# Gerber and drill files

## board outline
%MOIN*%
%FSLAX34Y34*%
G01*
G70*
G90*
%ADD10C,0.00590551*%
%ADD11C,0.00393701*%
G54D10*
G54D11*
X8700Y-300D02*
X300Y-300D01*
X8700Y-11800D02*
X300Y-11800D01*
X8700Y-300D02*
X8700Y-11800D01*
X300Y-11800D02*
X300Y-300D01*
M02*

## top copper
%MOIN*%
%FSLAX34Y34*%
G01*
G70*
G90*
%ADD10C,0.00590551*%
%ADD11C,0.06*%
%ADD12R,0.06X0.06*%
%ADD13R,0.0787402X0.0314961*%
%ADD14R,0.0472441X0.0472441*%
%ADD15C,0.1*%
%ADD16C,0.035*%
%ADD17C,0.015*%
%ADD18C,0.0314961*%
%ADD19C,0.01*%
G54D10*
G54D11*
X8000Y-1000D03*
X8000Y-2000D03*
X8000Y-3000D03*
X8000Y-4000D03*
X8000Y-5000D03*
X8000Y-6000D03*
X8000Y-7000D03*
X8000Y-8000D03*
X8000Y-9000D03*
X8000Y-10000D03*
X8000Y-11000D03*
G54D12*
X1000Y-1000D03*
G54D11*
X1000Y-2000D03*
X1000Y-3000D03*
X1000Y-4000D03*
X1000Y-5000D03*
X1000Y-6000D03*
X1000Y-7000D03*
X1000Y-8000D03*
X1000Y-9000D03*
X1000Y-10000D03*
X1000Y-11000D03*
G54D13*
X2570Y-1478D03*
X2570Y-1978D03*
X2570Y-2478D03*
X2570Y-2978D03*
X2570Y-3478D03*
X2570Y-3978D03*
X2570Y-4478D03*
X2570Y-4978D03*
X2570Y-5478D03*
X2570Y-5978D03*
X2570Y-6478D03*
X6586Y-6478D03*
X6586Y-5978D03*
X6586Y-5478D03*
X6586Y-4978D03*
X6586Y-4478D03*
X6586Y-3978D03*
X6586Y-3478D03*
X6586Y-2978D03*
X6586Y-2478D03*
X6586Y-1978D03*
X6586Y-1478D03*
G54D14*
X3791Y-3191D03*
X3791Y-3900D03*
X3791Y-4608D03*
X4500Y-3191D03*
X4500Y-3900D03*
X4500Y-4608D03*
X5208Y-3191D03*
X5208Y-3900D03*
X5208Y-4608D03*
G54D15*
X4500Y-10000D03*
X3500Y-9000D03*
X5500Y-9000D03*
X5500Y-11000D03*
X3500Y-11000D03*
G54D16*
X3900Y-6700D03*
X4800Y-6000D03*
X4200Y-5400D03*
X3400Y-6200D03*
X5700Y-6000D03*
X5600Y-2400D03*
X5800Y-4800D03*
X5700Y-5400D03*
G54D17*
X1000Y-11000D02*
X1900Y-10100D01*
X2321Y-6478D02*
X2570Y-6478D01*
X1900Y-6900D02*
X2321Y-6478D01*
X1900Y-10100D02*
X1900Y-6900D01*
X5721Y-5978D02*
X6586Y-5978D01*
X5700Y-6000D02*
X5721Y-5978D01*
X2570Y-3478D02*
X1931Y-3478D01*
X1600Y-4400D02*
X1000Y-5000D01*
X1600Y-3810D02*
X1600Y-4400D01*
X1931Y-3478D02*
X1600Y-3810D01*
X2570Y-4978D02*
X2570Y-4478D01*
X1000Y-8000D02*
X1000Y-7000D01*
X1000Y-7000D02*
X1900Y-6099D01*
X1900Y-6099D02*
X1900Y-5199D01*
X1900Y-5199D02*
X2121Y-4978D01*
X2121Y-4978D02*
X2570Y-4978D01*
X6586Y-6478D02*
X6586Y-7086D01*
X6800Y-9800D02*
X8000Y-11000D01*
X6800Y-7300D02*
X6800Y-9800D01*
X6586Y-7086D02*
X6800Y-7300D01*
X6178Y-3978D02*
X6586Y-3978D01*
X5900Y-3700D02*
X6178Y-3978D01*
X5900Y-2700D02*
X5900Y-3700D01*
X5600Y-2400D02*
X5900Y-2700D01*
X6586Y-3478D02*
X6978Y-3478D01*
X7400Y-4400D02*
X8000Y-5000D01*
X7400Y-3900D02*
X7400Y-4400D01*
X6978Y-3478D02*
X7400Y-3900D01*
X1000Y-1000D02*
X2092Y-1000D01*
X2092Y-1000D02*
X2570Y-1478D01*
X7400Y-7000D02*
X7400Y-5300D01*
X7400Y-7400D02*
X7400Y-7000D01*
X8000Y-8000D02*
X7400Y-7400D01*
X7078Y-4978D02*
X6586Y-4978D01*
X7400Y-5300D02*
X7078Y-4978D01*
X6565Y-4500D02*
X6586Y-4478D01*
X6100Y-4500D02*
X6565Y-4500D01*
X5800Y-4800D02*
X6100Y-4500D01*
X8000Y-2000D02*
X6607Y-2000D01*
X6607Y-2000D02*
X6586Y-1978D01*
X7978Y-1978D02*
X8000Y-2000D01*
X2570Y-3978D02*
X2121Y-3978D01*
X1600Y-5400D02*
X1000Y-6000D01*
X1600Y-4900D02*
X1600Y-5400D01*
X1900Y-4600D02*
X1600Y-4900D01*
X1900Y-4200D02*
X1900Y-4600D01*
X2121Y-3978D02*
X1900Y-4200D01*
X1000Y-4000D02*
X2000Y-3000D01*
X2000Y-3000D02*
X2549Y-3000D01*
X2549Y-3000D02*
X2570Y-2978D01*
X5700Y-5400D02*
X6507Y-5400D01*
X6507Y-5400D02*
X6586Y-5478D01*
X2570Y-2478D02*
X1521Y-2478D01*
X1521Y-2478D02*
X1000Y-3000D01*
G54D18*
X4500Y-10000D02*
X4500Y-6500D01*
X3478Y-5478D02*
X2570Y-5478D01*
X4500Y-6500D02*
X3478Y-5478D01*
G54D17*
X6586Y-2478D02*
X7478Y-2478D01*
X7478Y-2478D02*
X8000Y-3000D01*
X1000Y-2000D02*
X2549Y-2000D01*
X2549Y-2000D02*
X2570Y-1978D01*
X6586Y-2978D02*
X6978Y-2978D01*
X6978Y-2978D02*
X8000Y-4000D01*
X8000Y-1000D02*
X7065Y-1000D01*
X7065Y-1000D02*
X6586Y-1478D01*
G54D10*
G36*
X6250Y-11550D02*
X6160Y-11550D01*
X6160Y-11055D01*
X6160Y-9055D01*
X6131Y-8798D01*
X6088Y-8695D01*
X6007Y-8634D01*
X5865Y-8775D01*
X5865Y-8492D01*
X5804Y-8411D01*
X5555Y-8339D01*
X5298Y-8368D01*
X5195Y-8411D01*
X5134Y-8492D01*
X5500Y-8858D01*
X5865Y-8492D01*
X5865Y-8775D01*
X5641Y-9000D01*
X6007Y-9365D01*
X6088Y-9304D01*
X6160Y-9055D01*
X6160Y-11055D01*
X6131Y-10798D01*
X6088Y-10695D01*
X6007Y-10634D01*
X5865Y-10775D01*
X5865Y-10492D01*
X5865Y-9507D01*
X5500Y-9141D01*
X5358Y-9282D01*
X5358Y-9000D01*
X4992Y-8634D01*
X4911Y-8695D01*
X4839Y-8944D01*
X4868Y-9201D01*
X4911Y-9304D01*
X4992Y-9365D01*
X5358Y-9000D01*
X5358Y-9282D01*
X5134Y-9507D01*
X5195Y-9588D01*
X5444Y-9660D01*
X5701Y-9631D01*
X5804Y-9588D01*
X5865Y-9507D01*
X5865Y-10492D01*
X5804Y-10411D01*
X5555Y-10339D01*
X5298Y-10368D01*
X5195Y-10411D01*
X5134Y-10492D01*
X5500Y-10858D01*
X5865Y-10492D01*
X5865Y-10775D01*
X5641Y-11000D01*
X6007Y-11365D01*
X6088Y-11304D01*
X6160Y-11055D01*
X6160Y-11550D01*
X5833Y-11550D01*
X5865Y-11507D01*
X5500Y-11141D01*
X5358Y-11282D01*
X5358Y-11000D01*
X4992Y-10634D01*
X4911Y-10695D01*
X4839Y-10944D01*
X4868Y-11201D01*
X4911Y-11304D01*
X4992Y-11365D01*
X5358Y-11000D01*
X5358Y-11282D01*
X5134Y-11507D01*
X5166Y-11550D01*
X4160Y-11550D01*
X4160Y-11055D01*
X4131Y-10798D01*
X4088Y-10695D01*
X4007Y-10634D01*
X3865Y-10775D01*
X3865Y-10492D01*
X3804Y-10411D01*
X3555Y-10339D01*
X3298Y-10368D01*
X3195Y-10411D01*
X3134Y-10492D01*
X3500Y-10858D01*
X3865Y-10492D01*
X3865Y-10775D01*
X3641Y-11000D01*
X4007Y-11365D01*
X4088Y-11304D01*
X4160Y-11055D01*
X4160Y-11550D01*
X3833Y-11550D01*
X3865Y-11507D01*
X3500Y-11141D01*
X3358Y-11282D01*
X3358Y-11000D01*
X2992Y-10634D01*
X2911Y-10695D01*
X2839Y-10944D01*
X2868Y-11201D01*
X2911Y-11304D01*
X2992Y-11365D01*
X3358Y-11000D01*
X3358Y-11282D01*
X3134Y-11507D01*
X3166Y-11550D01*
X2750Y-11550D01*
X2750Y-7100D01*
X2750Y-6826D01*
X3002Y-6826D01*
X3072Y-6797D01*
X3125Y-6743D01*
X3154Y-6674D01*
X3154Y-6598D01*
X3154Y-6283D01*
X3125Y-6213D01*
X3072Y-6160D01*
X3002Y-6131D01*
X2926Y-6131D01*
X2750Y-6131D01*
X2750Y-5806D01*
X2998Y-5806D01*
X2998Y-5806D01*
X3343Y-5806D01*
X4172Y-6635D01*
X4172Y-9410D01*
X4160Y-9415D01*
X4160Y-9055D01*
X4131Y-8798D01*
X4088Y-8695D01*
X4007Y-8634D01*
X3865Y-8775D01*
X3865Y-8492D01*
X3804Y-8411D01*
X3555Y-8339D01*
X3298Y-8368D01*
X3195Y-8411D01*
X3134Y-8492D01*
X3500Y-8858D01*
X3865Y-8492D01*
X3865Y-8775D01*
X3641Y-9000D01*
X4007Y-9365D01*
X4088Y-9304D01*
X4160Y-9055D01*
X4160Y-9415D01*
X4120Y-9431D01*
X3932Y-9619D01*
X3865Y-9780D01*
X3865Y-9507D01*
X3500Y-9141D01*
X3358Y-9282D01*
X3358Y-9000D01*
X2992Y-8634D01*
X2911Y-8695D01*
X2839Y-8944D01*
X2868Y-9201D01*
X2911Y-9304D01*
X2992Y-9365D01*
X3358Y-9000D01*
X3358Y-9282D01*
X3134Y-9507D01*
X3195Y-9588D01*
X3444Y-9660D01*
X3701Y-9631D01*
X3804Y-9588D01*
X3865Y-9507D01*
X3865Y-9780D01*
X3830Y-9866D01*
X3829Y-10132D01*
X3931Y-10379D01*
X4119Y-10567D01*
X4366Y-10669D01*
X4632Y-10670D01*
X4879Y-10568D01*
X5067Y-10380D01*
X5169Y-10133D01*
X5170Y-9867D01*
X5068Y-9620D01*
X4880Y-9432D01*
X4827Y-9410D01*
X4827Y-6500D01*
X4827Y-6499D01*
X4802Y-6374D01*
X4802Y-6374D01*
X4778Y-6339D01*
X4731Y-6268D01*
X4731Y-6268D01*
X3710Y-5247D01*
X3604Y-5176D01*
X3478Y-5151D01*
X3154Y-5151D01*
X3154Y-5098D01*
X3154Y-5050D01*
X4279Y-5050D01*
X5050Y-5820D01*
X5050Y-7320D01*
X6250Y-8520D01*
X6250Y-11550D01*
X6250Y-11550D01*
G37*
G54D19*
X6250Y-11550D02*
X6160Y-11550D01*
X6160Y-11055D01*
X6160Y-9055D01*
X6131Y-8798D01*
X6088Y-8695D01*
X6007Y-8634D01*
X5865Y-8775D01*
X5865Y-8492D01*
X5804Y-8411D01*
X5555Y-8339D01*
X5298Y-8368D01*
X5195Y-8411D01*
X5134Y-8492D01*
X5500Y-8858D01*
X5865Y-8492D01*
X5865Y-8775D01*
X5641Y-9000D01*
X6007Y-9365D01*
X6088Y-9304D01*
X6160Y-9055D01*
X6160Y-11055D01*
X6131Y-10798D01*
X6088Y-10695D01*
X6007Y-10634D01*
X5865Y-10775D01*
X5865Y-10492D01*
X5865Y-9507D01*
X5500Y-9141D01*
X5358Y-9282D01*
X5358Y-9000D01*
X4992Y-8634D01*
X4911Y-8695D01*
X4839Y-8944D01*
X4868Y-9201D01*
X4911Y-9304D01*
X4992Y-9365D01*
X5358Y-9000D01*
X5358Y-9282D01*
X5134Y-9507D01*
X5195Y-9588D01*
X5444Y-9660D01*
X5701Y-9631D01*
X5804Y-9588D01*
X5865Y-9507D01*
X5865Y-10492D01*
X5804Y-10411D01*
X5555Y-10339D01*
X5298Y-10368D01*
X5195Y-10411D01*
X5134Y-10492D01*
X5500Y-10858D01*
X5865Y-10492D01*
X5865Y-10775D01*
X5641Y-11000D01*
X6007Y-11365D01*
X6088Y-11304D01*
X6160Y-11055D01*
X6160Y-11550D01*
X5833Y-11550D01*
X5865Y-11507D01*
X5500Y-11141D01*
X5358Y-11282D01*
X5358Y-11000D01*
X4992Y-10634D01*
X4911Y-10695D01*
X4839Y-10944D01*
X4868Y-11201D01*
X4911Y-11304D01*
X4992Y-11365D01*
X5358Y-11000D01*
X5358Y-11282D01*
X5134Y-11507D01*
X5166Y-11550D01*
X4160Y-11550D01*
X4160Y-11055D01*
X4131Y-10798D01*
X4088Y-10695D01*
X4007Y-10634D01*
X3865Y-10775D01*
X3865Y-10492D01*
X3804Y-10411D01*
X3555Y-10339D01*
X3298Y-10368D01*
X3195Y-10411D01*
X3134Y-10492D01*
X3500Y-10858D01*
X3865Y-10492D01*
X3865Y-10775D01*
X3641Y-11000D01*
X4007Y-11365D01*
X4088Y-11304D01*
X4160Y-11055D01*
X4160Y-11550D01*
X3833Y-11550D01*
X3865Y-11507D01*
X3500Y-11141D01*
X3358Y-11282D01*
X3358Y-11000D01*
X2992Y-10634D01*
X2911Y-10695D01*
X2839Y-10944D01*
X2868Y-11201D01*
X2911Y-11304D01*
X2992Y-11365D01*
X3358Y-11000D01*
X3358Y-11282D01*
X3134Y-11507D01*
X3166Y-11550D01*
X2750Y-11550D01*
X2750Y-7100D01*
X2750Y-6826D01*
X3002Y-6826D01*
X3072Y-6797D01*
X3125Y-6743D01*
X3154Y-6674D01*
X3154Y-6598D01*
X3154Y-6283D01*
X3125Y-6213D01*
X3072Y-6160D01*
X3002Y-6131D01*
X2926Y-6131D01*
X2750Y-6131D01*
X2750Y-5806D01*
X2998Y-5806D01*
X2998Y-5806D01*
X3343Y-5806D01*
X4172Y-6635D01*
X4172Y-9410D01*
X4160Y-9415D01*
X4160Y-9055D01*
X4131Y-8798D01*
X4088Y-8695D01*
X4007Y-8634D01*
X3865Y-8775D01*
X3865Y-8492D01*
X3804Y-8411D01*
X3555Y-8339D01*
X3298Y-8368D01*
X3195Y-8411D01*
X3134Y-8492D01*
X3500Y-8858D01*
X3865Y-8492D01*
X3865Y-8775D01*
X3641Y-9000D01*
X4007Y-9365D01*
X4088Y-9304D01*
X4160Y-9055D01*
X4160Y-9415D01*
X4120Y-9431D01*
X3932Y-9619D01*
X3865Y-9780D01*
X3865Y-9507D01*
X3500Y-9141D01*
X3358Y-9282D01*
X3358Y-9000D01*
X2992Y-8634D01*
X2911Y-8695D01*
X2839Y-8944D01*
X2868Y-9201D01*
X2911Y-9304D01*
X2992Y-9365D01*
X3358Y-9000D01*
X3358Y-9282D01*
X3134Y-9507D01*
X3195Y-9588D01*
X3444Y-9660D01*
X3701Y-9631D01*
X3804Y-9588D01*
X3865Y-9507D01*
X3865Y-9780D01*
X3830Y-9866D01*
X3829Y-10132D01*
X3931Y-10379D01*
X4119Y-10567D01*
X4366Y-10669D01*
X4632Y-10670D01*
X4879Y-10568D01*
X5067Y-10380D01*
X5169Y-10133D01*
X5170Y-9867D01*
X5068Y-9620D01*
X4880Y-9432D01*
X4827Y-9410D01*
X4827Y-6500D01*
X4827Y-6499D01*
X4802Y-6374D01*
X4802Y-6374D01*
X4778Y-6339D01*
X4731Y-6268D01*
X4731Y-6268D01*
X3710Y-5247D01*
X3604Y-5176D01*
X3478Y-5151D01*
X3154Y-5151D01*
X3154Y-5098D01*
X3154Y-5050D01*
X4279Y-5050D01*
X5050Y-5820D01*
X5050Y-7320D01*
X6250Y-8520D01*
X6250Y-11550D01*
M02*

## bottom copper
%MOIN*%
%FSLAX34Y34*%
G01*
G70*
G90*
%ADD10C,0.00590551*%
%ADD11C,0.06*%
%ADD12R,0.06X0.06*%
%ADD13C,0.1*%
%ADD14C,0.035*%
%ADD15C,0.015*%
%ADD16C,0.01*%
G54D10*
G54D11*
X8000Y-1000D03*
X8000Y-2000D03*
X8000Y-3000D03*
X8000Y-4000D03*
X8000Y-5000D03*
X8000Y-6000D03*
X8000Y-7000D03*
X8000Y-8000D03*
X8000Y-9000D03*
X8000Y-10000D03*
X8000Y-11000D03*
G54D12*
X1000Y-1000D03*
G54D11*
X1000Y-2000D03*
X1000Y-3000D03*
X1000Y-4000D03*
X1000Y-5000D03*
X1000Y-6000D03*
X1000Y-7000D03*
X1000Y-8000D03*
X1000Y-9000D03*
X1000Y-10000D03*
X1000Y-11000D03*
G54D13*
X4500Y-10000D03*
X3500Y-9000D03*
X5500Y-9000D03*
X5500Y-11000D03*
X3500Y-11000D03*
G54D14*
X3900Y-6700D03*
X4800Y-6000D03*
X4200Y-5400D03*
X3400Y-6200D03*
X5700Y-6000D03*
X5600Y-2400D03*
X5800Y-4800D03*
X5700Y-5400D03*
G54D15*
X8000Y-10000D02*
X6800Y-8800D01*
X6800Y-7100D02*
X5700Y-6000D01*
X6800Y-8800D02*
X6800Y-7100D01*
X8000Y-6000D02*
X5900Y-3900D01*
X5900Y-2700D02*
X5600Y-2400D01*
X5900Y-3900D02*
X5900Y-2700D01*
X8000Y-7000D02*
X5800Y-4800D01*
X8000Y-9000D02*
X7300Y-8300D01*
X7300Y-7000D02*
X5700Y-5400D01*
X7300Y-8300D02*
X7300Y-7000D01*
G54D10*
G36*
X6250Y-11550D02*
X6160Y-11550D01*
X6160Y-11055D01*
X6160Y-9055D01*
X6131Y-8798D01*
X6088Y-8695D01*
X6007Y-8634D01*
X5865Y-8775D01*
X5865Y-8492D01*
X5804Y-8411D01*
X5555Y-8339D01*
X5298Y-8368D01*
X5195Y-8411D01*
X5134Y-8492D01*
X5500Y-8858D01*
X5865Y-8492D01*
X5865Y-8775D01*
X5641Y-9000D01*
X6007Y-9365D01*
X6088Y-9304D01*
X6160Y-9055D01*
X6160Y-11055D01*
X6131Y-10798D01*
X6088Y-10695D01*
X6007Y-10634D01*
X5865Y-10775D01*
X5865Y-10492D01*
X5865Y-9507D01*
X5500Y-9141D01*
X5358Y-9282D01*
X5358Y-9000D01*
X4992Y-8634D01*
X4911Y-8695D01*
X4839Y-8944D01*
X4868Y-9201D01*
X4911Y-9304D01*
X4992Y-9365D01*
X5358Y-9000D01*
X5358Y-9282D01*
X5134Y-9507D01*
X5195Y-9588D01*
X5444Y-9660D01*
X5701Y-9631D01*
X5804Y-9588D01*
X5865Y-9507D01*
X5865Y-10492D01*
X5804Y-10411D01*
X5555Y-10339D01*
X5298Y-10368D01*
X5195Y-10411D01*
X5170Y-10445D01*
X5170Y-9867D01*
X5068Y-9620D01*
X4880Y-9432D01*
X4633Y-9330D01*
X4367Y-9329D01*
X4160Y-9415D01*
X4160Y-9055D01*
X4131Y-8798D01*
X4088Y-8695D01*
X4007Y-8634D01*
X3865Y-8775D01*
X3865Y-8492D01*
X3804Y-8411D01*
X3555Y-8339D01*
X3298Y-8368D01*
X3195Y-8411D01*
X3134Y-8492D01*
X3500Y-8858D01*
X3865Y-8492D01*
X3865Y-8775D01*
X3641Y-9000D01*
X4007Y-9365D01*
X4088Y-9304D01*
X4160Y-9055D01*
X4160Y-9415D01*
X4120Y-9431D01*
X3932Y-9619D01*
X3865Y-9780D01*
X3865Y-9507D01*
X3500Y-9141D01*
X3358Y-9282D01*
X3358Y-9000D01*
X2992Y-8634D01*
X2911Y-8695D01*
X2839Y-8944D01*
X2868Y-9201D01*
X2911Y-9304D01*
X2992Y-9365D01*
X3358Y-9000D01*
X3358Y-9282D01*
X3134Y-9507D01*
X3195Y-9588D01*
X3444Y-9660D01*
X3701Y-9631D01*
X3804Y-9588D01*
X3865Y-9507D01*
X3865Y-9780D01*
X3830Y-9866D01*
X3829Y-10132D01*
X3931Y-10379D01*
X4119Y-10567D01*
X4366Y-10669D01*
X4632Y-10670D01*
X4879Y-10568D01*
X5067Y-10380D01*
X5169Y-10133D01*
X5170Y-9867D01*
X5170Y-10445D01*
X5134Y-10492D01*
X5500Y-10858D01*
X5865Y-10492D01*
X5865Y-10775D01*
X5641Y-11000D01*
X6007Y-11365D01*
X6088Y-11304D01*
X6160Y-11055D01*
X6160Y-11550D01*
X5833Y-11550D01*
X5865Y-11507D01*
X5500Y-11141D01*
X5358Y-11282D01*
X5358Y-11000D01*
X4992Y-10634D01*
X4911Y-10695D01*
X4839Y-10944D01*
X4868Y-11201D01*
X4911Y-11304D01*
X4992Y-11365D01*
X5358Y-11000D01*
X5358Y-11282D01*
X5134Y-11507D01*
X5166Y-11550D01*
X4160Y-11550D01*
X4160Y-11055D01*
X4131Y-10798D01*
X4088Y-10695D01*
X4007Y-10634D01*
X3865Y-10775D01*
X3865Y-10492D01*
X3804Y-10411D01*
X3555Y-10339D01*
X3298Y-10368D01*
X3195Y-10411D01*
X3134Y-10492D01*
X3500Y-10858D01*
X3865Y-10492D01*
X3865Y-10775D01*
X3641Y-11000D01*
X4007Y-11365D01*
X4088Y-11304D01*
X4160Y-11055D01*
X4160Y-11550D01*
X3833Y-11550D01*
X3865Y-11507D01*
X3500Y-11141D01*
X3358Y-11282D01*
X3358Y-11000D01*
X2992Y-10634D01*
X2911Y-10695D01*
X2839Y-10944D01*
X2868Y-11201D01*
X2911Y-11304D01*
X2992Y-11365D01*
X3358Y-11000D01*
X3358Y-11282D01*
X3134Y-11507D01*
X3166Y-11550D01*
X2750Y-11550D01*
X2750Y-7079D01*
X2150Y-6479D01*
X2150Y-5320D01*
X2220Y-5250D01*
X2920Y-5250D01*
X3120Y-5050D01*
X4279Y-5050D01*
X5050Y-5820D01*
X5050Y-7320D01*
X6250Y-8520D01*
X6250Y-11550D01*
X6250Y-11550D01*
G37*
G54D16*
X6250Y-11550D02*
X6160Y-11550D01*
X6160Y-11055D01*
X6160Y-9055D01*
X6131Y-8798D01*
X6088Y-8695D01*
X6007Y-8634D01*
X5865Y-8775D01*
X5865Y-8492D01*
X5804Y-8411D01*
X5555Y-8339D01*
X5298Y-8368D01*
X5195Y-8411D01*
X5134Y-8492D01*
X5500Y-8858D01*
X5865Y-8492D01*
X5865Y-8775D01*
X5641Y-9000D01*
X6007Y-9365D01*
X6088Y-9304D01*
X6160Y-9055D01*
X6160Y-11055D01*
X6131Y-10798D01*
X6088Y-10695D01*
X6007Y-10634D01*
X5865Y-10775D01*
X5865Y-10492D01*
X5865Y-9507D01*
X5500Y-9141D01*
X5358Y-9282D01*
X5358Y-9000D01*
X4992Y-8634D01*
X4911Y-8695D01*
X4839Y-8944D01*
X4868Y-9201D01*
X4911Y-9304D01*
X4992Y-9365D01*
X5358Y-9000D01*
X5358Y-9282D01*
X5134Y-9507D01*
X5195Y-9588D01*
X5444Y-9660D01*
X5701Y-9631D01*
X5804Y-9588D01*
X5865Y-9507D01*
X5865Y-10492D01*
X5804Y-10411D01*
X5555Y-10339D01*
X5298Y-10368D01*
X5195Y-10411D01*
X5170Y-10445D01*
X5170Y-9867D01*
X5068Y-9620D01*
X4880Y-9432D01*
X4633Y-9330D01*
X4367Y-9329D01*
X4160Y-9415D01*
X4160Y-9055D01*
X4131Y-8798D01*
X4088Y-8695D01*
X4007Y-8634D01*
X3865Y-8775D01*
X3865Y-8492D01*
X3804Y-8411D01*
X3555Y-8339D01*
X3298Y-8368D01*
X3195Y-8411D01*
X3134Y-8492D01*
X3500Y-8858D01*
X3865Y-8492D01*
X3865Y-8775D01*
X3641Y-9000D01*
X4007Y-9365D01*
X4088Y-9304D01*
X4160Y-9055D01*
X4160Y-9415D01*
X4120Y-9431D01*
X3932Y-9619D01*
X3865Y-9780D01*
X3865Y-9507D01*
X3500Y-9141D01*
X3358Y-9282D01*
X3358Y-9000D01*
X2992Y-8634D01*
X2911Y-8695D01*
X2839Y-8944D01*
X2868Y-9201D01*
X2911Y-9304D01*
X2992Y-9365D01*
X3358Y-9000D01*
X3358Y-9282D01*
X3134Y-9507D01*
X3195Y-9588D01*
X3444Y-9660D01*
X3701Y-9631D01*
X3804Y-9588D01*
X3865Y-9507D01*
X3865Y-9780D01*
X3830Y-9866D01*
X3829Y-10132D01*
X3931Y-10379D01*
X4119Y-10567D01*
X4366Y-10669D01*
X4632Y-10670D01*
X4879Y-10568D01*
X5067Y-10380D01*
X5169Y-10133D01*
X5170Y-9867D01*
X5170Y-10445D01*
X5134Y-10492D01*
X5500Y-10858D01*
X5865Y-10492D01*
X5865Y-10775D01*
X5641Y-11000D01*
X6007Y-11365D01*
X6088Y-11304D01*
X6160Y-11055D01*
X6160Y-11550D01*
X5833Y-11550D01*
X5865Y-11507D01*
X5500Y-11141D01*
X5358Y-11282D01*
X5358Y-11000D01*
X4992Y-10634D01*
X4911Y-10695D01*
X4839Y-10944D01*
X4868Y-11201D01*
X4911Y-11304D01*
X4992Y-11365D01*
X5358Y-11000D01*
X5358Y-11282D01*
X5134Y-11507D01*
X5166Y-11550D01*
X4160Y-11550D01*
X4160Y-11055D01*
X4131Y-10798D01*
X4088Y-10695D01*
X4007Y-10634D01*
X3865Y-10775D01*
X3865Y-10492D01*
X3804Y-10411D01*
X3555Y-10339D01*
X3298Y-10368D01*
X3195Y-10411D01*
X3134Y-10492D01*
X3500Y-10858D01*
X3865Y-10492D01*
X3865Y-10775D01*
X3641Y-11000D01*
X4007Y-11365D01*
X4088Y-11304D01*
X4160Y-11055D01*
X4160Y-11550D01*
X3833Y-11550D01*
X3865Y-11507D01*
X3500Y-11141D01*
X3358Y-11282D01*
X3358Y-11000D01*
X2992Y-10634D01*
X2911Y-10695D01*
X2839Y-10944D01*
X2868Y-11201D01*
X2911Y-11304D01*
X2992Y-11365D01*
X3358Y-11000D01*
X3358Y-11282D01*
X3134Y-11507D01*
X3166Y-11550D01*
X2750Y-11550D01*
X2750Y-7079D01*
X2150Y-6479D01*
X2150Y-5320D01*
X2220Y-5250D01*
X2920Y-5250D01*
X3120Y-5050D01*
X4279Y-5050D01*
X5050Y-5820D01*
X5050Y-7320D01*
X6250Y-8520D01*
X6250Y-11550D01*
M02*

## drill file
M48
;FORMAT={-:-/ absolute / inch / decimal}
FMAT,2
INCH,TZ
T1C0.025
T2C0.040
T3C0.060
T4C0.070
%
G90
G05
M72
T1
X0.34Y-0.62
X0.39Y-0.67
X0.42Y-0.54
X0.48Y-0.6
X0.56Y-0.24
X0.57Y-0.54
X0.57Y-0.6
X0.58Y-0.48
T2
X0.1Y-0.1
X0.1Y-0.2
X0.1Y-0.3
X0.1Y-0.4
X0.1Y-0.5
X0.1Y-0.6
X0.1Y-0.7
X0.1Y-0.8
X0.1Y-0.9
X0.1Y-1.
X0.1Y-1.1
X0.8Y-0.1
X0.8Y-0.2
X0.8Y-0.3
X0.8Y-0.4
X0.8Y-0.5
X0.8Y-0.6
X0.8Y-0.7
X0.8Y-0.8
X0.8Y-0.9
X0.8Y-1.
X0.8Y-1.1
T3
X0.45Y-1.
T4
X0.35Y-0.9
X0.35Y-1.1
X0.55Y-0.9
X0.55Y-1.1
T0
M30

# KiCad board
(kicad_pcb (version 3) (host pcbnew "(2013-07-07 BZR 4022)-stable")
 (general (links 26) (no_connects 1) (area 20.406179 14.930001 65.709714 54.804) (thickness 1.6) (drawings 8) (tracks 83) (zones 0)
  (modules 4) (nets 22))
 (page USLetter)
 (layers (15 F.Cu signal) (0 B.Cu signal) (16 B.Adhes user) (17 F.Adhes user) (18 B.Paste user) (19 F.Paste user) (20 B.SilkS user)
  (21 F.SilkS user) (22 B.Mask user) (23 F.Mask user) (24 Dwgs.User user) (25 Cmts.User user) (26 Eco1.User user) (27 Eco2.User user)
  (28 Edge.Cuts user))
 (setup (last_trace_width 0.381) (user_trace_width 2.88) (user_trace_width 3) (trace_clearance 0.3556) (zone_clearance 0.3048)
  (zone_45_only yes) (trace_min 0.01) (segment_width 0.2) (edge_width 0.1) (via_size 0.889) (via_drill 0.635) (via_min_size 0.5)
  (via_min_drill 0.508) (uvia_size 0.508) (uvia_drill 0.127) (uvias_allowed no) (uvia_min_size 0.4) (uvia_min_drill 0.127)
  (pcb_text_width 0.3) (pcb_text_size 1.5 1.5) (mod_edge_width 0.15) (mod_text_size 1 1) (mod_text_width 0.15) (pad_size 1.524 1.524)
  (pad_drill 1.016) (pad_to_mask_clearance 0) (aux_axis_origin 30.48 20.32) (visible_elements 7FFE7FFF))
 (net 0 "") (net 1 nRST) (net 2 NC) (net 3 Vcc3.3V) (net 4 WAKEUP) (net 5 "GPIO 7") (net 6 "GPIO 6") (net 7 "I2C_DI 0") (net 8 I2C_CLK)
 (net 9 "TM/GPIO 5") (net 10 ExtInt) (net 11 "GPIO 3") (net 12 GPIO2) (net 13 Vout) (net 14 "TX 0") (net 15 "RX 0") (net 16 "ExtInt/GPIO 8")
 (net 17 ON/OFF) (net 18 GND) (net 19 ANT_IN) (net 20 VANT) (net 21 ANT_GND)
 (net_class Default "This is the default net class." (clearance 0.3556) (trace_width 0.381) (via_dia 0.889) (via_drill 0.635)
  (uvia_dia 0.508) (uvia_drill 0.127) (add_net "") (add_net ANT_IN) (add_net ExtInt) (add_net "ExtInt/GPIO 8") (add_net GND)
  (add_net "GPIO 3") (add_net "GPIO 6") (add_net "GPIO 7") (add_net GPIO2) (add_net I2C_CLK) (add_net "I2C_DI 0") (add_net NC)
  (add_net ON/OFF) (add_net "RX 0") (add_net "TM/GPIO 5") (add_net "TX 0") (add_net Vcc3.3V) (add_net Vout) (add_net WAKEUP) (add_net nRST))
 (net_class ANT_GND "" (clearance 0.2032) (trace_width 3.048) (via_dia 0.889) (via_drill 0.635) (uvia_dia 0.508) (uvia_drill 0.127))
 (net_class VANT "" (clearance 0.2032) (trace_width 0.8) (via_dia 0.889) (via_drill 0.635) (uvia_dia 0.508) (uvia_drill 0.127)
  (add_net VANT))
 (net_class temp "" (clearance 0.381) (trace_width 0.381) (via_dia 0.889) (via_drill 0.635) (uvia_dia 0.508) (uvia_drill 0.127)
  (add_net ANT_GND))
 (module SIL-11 (layer F.Cu) (at 50.8 35.56 270)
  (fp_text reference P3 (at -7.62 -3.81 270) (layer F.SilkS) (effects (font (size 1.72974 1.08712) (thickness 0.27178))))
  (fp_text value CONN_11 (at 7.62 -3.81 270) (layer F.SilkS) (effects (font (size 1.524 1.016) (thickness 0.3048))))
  (pad 1 thru_hole circle (at -12.7 0 270) (size 1.524 1.524) (drill 1.016) (layers *.Cu *.Mask F.SilkS) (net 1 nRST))
  (pad 2 thru_hole circle (at -10.16 0 270) (size 1.524 1.524) (drill 1.016) (layers *.Cu *.Mask F.SilkS) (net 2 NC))
  (pad 3 thru_hole circle (at -7.62 0 270) (size 1.524 1.524) (drill 1.016) (layers *.Cu *.Mask F.SilkS) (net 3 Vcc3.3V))
  (pad 4 thru_hole circle (at -5.08 0 270) (size 1.524 1.524) (drill 1.016) (layers *.Cu *.Mask F.SilkS) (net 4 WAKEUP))
  (pad 5 thru_hole circle (at -2.54 0 270) (size 1.524 1.524) (drill 1.016) (layers *.Cu *.Mask F.SilkS) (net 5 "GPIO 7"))
  (pad 6 thru_hole circle (at 0 0 270) (size 1.524 1.524) (drill 1.016) (layers *.Cu *.Mask F.SilkS) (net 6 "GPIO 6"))
  (pad 7 thru_hole circle (at 2.54 0 270) (size 1.524 1.524) (drill 1.016) (layers *.Cu *.Mask F.SilkS) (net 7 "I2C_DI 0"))
  (pad 8 thru_hole circle (at 5.08 0 270) (size 1.524 1.524) (drill 1.016) (layers *.Cu *.Mask F.SilkS) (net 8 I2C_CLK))
  (pad 9 thru_hole circle (at 7.62 0 270) (size 1.524 1.524) (drill 1.016) (layers *.Cu *.Mask F.SilkS) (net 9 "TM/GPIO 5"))
  (pad 10 thru_hole circle (at 10.16 0 270) (size 1.524 1.524) (drill 1.016) (layers *.Cu *.Mask F.SilkS) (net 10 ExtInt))
  (pad 11 thru_hole circle (at 12.7 0 270) (size 1.524 1.524) (drill 1.016) (layers *.Cu *.Mask F.SilkS) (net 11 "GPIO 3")))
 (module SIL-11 (layer F.Cu) (at 33.02 35.56 270)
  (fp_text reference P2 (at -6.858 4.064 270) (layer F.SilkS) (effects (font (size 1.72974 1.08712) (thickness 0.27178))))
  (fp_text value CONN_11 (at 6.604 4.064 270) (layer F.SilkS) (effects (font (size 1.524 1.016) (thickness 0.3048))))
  (pad 1 thru_hole rect (at -12.7 0 270) (size 1.524 1.524) (drill 1.016) (layers *.Cu *.Mask F.SilkS) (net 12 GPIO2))
  (pad 2 thru_hole circle (at -10.16 0 270) (size 1.524 1.524) (drill 1.016) (layers *.Cu *.Mask F.SilkS) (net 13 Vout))
  (pad 3 thru_hole circle (at -7.62 0 270) (size 1.524 1.524) (drill 1.016) (layers *.Cu *.Mask F.SilkS) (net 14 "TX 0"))
  (pad 4 thru_hole circle (at -5.08 0 270) (size 1.524 1.524) (drill 1.016) (layers *.Cu *.Mask F.SilkS) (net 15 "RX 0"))
  (pad 5 thru_hole circle (at -2.54 0 270) (size 1.524 1.524) (drill 1.016) (layers *.Cu *.Mask F.SilkS) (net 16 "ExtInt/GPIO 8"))
  (pad 6 thru_hole circle (at 0 0 270) (size 1.524 1.524) (drill 1.016) (layers *.Cu *.Mask F.SilkS) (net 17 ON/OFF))
  (pad 7 thru_hole circle (at 2.54 0 270) (size 1.524 1.524) (drill 1.016) (layers *.Cu *.Mask F.SilkS) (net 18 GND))
  (pad 8 thru_hole circle (at 5.08 0 270) (size 1.524 1.524) (drill 1.016) (layers *.Cu *.Mask F.SilkS) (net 18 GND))
  (pad 9 thru_hole circle (at 7.62 0 270) (size 1.524 1.524) (drill 1.016) (layers *.Cu *.Mask F.SilkS))
  (pad 10 thru_hole circle (at 10.16 0 270) (size 1.524 1.524) (drill 1.016) (layers *.Cu *.Mask F.SilkS))
  (pad 11 thru_hole circle (at 12.7 0 270) (size 1.524 1.524) (drill 1.016) (layers *.Cu *.Mask F.SilkS) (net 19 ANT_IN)))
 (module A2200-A (layer F.Cu) (at 41.91 30.226)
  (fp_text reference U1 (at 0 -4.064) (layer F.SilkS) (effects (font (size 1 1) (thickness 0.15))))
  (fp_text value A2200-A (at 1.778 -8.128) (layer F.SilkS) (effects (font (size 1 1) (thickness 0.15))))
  (pad 1 smd rect (at -4.9 -6.15) (size 2 0.8) (layers F.Cu F.Paste F.Mask) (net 12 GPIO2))
  (pad 2 smd rect (at -4.9 -4.88) (size 2 0.8) (layers F.Cu F.Paste F.Mask) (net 13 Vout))
  (pad 3 smd rect (at -4.9 -3.61) (size 2 0.8) (layers F.Cu F.Paste F.Mask) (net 14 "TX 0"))
  (pad 4 smd rect (at -4.9 -2.34) (size 2 0.8) (layers F.Cu F.Paste F.Mask) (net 15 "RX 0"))
  (pad 5 smd rect (at -4.9 -1.07) (size 2 0.8) (layers F.Cu F.Paste F.Mask) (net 16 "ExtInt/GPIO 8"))
  (pad 6 smd rect (at -4.9 0.2) (size 2 0.8) (layers F.Cu F.Paste F.Mask) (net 17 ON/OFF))
  (pad 7 smd rect (at -4.9 1.47) (size 2 0.8) (layers F.Cu F.Paste F.Mask) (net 18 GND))
  (pad 8 smd rect (at -4.9 2.74) (size 2 0.8) (layers F.Cu F.Paste F.Mask) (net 18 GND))
  (pad 9 smd rect (at -4.9 4.01) (size 2 0.8) (layers F.Cu F.Paste F.Mask) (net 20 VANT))
  (pad 10 smd rect (at -4.9 5.28) (size 2 0.8) (layers F.Cu F.Paste F.Mask) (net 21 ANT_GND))
  (pad 11 smd rect (at -4.9 6.55) (size 2 0.8) (layers F.Cu F.Paste F.Mask) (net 19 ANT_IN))
  (pad 12 smd rect (at 5.3 6.55) (size 2 0.8) (layers F.Cu F.Paste F.Mask) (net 11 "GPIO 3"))
  (pad 13 smd rect (at 5.3 5.28) (size 2 0.8) (layers F.Cu F.Paste F.Mask) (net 10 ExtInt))
  (pad 14 smd rect (at 5.3 4.01) (size 2 0.8) (layers F.Cu F.Paste F.Mask) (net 9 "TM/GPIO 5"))
  (pad 15 smd rect (at 5.3 2.74) (size 2 0.8) (layers F.Cu F.Paste F.Mask) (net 8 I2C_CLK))
  (pad 16 smd rect (at 5.3 1.47) (size 2 0.8) (layers F.Cu F.Paste F.Mask) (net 7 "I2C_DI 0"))
  (pad 17 smd rect (at 5.3 0.2) (size 2 0.8) (layers F.Cu F.Paste F.Mask) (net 6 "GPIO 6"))
  (pad 18 smd rect (at 5.3 -1.07) (size 2 0.8) (layers F.Cu F.Paste F.Mask) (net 5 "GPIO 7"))
  (pad 19 smd rect (at 5.3 -2.34) (size 2 0.8) (layers F.Cu F.Paste F.Mask) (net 4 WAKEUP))
  (pad 20 smd rect (at 5.3 -3.61) (size 2 0.8) (layers F.Cu F.Paste F.Mask) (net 3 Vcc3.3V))
  (pad 21 smd rect (at 5.3 -4.88) (size 2 0.8) (layers F.Cu F.Paste F.Mask) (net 2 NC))
  (pad 22 smd rect (at 5.3 -6.15) (size 2 0.8) (layers F.Cu F.Paste F.Mask) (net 1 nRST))
  (pad 23 smd rect (at -1.8 -1.8) (size 1.2 1.2) (layers F.Cu F.Paste F.Mask))
  (pad 24 smd rect (at -1.8 0) (size 1.2 1.2) (layers F.Cu F.Paste F.Mask))
  (pad 25 smd rect (at -1.8 1.8) (size 1.2 1.2) (layers F.Cu F.Paste F.Mask))
  (pad 26 smd rect (at 0 -1.8) (size 1.2 1.2) (layers F.Cu F.Paste F.Mask))
  (pad 27 smd rect (at 0 0) (size 1.2 1.2) (layers F.Cu F.Paste F.Mask))
  (pad 29 smd rect (at 0 1.8) (size 1.2 1.2) (layers F.Cu F.Paste F.Mask))
  (pad 30 smd rect (at 1.8 -1.8) (size 1.2 1.2) (layers F.Cu F.Paste F.Mask))
  (pad 31 smd rect (at 1.8 0) (size 1.2 1.2) (layers F.Cu F.Paste F.Mask))
  (pad 32 smd rect (at 1.8 1.8) (size 1.2 1.2) (layers F.Cu F.Paste F.Mask)))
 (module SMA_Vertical (layer F.Cu) (at 41.91 45.72)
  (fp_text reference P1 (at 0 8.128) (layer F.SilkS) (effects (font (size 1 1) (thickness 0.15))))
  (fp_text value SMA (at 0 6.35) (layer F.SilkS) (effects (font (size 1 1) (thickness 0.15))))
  (pad 1 thru_hole circle (at 0 0) (size 2.54 2.54) (drill 1.524) (layers *.Cu *.Mask F.SilkS) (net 20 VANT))
  (pad 2 thru_hole circle (at -2.54 -2.54) (size 2.54 2.54) (drill 1.778) (layers *.Cu *.Mask F.SilkS) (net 21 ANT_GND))
  (pad 2 thru_hole circle (at 2.54 -2.54) (size 2.54 2.54) (drill 1.778) (layers *.Cu *.Mask F.SilkS) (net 21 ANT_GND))
  (pad 2 thru_hole circle (at 2.54 2.54) (size 2.54 2.54) (drill 1.778) (layers *.Cu *.Mask F.SilkS) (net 21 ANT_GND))
  (pad 2 thru_hole circle (at -2.54 2.54) (size 2.54 2.54) (drill 1.778) (layers *.Cu *.Mask F.SilkS) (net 21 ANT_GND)))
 (gr_line (start 52.578 21.082) (end 31.242 21.082) (angle 90) (layer Edge.Cuts) (width 0.1))
 (gr_line (start 52.578 50.292) (end 31.242 50.292) (angle 90) (layer Edge.Cuts) (width 0.1))
 (gr_line (start 52.578 21.082) (end 52.578 50.292) (angle 90) (layer Edge.Cuts) (width 0.1))
 (gr_line (start 31.242 50.292) (end 31.242 21.082) (angle 90) (layer Edge.Cuts) (width 0.1))
 (via (at 40.386 37.338) (size 0.889) (layers F.Cu B.Cu) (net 21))
 (via (at 42.672 35.56) (size 0.889) (layers F.Cu B.Cu) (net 21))
 (via (at 41.148 34.036) (size 0.889) (layers F.Cu B.Cu) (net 21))
 (via (at 39.116 36.068) (size 0.889) (layers F.Cu B.Cu) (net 21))
 (segment (start 33.02 48.26) (end 35.306 45.974) (width 0.381) (layer F.Cu) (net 19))
 (segment (start 36.376 36.776) (end 37.01 36.776) (width 0.381) (layer F.Cu) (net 19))
 (segment (start 35.306 37.846) (end 36.376 36.776) (width 0.381) (layer F.Cu) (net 19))
 (segment (start 35.306 45.974) (end 35.306 37.846) (width 0.381) (layer F.Cu) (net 19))
 (segment (start 50.8 45.72) (end 47.752 42.672) (width 0.381) (layer B.Cu) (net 10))
 (segment (start 45.012 35.506) (end 47.21 35.506) (width 0.381) (layer F.Cu) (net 10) (status 800000))
 (segment (start 44.958 35.56) (end 45.012 35.506) (width 0.381) (layer F.Cu) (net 10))
 (via (at 44.958 35.56) (size 0.889) (layers F.Cu B.Cu) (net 10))
 (segment (start 47.752 38.354) (end 44.958 35.56) (width 0.381) (layer B.Cu) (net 10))
 (segment (start 47.752 42.672) (end 47.752 38.354) (width 0.381) (layer B.Cu) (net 10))
 (segment (start 37.01 29.156) (end 35.385712 29.156) (width 0.381) (layer F.Cu) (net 16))
 (segment (start 34.544 31.496) (end 33.02 33.02) (width 0.381) (layer F.Cu) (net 16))
 (segment (start 34.544 29.997712) (end 34.544 31.496) (width 0.381) (layer F.Cu) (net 16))
 (segment (start 35.385712 29.156) (end 34.544 29.997712) (width 0.381) (layer F.Cu) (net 16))
 (segment (start 37.01 32.966) (end 37.01 31.696) (width 0.381) (layer F.Cu) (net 18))
 (segment (start 33.02 40.64) (end 33.02 38.1) (width 0.381) (layer F.Cu) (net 18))
 (segment (start 33.02 38.1) (end 35.306 35.813998) (width 0.381) (layer F.Cu) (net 18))
 (segment (start 35.306 35.813998) (end 35.306 33.527998) (width 0.381) (layer F.Cu) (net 18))
 (segment (start 35.306 33.527998) (end 35.868 32.966) (width 0.381) (layer F.Cu) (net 18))
 (segment (start 35.868 32.966) (end 37.01 32.966) (width 0.381) (layer F.Cu) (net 18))
 (segment (start 47.21 36.776) (end 47.21 38.32) (width 0.381) (layer F.Cu) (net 11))
 (segment (start 47.752 45.212) (end 50.8 48.26) (width 0.381) (layer F.Cu) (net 11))
 (segment (start 47.752 38.862) (end 47.752 45.212) (width 0.381) (layer F.Cu) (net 11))
 (segment (start 47.21 38.32) (end 47.752 38.862) (width 0.381) (layer F.Cu) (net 11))
 (segment (start 50.8 35.56) (end 45.466 30.226) (width 0.381) (layer B.Cu) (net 6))
 (segment (start 46.174 30.426) (end 47.21 30.426) (width 0.381) (layer F.Cu) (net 6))
 (segment (start 45.466 29.718) (end 46.174 30.426) (width 0.381) (layer F.Cu) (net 6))
 (segment (start 45.466 27.178) (end 45.466 29.718) (width 0.381) (layer F.Cu) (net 6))
 (segment (start 44.704 26.416) (end 45.466 27.178) (width 0.381) (layer F.Cu) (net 6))
 (via (at 44.704 26.416) (size 0.889) (layers F.Cu B.Cu) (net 6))
 (segment (start 45.466 27.178) (end 44.704 26.416) (width 0.381) (layer B.Cu) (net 6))
 (segment (start 45.466 30.226) (end 45.466 27.178) (width 0.381) (layer B.Cu) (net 6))
 (segment (start 47.21 29.156) (end 48.206 29.156) (width 0.381) (layer F.Cu) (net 5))
 (segment (start 49.276 31.496) (end 50.8 33.02) (width 0.381) (layer F.Cu) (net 5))
 (segment (start 49.276 30.226) (end 49.276 31.496) (width 0.381) (layer F.Cu) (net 5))
 (segment (start 48.206 29.156) (end 49.276 30.226) (width 0.381) (layer F.Cu) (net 5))
 (segment (start 33.02 22.86) (end 35.794 22.86) (width 0.381) (layer F.Cu) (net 12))
 (segment (start 35.794 22.86) (end 37.01 24.076) (width 0.381) (layer F.Cu) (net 12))
 (segment (start 49.276 38.1) (end 49.276 33.782) (width 0.381) (layer F.Cu) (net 8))
 (segment (start 49.276 39.116) (end 49.276 38.1) (width 0.381) (layer F.Cu) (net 8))
 (segment (start 50.8 40.64) (end 49.276 39.116) (width 0.381) (layer F.Cu) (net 8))
 (segment (start 48.46 32.966) (end 47.21 32.966) (width 0.381) (layer F.Cu) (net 8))
 (segment (start 49.276 33.782) (end 48.46 32.966) (width 0.381) (layer F.Cu) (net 8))
 (segment (start 50.8 38.1) (end 45.212 32.512) (width 0.381) (layer B.Cu) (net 7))
 (segment (start 47.156 31.75) (end 47.21 31.696) (width 0.381) (layer F.Cu) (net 7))
 (segment (start 45.974 31.75) (end 47.156 31.75) (width 0.381) (layer F.Cu) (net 7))
 (segment (start 45.212 32.512) (end 45.974 31.75) (width 0.381) (layer F.Cu) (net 7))
 (via (at 45.212 32.512) (size 0.889) (layers F.Cu B.Cu) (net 7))
 (segment (start 50.8 25.4) (end 47.264 25.4) (width 0.381) (layer F.Cu) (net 2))
 (segment (start 47.264 25.4) (end 47.21 25.346) (width 0.381) (layer F.Cu) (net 2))
 (segment (start 50.746 25.346) (end 50.8 25.4) (width 0.381) (layer F.Cu) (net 2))
 (segment (start 37.01 30.426) (end 35.868 30.426) (width 0.381) (layer F.Cu) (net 17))
 (segment (start 34.544 34.036) (end 33.02 35.56) (width 0.381) (layer F.Cu) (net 17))
 (segment (start 34.544 32.766) (end 34.544 34.036) (width 0.381) (layer F.Cu) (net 17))
 (segment (start 35.306 32.004) (end 34.544 32.766) (width 0.381) (layer F.Cu) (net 17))
 (segment (start 35.306 30.988) (end 35.306 32.004) (width 0.381) (layer F.Cu) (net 17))
 (segment (start 35.868 30.426) (end 35.306 30.988) (width 0.381) (layer F.Cu) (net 17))
 (segment (start 33.02 30.48) (end 35.56 27.94) (width 0.381) (layer F.Cu) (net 15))
 (segment (start 35.56 27.94) (end 36.956 27.94) (width 0.381) (layer F.Cu) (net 15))
 (segment (start 36.956 27.94) (end 37.01 27.886) (width 0.381) (layer F.Cu) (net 15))
 (segment (start 44.958 34.036) (end 47.01 34.036) (width 0.381) (layer F.Cu) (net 9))
 (segment (start 47.01 34.036) (end 47.21 34.236) (width 0.381) (layer F.Cu) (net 9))
 (segment (start 50.8 43.18) (end 49.022 41.402) (width 0.381) (layer B.Cu) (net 9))
 (via (at 44.958 34.036) (size 0.889) (layers F.Cu B.Cu) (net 9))
 (segment (start 49.022 38.1) (end 44.958 34.036) (width 0.381) (layer B.Cu) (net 9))
 (segment (start 49.022 41.402) (end 49.022 38.1) (width 0.381) (layer B.Cu) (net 9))
 (segment (start 37.01 26.616) (end 34.344 26.616) (width 0.381) (layer F.Cu) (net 14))
 (segment (start 34.344 26.616) (end 33.02 27.94) (width 0.381) (layer F.Cu) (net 14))
 (segment (start 41.91 45.72) (end 41.91 36.83) (width 0.8) (layer F.Cu) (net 20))
 (segment (start 39.316 34.236) (end 37.01 34.236) (width 0.8) (layer F.Cu) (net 20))
 (segment (start 41.91 36.83) (end 39.316 34.236) (width 0.8) (layer F.Cu) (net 20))
 (segment (start 47.21 26.616) (end 49.476 26.616) (width 0.381) (layer F.Cu) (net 3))
 (segment (start 49.476 26.616) (end 50.8 27.94) (width 0.381) (layer F.Cu) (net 3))
 (segment (start 33.02 25.4) (end 36.956 25.4) (width 0.381) (layer F.Cu) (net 13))
 (segment (start 36.956 25.4) (end 37.01 25.346) (width 0.381) (layer F.Cu) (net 13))
 (segment (start 47.21 27.886) (end 48.206 27.886) (width 0.381) (layer F.Cu) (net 4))
 (segment (start 48.206 27.886) (end 50.8 30.48) (width 0.381) (layer F.Cu) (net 4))
 (segment (start 50.8 22.86) (end 48.426 22.86) (width 0.381) (layer F.Cu) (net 1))
 (segment (start 48.426 22.86) (end 47.21 24.076) (width 0.381) (layer F.Cu) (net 1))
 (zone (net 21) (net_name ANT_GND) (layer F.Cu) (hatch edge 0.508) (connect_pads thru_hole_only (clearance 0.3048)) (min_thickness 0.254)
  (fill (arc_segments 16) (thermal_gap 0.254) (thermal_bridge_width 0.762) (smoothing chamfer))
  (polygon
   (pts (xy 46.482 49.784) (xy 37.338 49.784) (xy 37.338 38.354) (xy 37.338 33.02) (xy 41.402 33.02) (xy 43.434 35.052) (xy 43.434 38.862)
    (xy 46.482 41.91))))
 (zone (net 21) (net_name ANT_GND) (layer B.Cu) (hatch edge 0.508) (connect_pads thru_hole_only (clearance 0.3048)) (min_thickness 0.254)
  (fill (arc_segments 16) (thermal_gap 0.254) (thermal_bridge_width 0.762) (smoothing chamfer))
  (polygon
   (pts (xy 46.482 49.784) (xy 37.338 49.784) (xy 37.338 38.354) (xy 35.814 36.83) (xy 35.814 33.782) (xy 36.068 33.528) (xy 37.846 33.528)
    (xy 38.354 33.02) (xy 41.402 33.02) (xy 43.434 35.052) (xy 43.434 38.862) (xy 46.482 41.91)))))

